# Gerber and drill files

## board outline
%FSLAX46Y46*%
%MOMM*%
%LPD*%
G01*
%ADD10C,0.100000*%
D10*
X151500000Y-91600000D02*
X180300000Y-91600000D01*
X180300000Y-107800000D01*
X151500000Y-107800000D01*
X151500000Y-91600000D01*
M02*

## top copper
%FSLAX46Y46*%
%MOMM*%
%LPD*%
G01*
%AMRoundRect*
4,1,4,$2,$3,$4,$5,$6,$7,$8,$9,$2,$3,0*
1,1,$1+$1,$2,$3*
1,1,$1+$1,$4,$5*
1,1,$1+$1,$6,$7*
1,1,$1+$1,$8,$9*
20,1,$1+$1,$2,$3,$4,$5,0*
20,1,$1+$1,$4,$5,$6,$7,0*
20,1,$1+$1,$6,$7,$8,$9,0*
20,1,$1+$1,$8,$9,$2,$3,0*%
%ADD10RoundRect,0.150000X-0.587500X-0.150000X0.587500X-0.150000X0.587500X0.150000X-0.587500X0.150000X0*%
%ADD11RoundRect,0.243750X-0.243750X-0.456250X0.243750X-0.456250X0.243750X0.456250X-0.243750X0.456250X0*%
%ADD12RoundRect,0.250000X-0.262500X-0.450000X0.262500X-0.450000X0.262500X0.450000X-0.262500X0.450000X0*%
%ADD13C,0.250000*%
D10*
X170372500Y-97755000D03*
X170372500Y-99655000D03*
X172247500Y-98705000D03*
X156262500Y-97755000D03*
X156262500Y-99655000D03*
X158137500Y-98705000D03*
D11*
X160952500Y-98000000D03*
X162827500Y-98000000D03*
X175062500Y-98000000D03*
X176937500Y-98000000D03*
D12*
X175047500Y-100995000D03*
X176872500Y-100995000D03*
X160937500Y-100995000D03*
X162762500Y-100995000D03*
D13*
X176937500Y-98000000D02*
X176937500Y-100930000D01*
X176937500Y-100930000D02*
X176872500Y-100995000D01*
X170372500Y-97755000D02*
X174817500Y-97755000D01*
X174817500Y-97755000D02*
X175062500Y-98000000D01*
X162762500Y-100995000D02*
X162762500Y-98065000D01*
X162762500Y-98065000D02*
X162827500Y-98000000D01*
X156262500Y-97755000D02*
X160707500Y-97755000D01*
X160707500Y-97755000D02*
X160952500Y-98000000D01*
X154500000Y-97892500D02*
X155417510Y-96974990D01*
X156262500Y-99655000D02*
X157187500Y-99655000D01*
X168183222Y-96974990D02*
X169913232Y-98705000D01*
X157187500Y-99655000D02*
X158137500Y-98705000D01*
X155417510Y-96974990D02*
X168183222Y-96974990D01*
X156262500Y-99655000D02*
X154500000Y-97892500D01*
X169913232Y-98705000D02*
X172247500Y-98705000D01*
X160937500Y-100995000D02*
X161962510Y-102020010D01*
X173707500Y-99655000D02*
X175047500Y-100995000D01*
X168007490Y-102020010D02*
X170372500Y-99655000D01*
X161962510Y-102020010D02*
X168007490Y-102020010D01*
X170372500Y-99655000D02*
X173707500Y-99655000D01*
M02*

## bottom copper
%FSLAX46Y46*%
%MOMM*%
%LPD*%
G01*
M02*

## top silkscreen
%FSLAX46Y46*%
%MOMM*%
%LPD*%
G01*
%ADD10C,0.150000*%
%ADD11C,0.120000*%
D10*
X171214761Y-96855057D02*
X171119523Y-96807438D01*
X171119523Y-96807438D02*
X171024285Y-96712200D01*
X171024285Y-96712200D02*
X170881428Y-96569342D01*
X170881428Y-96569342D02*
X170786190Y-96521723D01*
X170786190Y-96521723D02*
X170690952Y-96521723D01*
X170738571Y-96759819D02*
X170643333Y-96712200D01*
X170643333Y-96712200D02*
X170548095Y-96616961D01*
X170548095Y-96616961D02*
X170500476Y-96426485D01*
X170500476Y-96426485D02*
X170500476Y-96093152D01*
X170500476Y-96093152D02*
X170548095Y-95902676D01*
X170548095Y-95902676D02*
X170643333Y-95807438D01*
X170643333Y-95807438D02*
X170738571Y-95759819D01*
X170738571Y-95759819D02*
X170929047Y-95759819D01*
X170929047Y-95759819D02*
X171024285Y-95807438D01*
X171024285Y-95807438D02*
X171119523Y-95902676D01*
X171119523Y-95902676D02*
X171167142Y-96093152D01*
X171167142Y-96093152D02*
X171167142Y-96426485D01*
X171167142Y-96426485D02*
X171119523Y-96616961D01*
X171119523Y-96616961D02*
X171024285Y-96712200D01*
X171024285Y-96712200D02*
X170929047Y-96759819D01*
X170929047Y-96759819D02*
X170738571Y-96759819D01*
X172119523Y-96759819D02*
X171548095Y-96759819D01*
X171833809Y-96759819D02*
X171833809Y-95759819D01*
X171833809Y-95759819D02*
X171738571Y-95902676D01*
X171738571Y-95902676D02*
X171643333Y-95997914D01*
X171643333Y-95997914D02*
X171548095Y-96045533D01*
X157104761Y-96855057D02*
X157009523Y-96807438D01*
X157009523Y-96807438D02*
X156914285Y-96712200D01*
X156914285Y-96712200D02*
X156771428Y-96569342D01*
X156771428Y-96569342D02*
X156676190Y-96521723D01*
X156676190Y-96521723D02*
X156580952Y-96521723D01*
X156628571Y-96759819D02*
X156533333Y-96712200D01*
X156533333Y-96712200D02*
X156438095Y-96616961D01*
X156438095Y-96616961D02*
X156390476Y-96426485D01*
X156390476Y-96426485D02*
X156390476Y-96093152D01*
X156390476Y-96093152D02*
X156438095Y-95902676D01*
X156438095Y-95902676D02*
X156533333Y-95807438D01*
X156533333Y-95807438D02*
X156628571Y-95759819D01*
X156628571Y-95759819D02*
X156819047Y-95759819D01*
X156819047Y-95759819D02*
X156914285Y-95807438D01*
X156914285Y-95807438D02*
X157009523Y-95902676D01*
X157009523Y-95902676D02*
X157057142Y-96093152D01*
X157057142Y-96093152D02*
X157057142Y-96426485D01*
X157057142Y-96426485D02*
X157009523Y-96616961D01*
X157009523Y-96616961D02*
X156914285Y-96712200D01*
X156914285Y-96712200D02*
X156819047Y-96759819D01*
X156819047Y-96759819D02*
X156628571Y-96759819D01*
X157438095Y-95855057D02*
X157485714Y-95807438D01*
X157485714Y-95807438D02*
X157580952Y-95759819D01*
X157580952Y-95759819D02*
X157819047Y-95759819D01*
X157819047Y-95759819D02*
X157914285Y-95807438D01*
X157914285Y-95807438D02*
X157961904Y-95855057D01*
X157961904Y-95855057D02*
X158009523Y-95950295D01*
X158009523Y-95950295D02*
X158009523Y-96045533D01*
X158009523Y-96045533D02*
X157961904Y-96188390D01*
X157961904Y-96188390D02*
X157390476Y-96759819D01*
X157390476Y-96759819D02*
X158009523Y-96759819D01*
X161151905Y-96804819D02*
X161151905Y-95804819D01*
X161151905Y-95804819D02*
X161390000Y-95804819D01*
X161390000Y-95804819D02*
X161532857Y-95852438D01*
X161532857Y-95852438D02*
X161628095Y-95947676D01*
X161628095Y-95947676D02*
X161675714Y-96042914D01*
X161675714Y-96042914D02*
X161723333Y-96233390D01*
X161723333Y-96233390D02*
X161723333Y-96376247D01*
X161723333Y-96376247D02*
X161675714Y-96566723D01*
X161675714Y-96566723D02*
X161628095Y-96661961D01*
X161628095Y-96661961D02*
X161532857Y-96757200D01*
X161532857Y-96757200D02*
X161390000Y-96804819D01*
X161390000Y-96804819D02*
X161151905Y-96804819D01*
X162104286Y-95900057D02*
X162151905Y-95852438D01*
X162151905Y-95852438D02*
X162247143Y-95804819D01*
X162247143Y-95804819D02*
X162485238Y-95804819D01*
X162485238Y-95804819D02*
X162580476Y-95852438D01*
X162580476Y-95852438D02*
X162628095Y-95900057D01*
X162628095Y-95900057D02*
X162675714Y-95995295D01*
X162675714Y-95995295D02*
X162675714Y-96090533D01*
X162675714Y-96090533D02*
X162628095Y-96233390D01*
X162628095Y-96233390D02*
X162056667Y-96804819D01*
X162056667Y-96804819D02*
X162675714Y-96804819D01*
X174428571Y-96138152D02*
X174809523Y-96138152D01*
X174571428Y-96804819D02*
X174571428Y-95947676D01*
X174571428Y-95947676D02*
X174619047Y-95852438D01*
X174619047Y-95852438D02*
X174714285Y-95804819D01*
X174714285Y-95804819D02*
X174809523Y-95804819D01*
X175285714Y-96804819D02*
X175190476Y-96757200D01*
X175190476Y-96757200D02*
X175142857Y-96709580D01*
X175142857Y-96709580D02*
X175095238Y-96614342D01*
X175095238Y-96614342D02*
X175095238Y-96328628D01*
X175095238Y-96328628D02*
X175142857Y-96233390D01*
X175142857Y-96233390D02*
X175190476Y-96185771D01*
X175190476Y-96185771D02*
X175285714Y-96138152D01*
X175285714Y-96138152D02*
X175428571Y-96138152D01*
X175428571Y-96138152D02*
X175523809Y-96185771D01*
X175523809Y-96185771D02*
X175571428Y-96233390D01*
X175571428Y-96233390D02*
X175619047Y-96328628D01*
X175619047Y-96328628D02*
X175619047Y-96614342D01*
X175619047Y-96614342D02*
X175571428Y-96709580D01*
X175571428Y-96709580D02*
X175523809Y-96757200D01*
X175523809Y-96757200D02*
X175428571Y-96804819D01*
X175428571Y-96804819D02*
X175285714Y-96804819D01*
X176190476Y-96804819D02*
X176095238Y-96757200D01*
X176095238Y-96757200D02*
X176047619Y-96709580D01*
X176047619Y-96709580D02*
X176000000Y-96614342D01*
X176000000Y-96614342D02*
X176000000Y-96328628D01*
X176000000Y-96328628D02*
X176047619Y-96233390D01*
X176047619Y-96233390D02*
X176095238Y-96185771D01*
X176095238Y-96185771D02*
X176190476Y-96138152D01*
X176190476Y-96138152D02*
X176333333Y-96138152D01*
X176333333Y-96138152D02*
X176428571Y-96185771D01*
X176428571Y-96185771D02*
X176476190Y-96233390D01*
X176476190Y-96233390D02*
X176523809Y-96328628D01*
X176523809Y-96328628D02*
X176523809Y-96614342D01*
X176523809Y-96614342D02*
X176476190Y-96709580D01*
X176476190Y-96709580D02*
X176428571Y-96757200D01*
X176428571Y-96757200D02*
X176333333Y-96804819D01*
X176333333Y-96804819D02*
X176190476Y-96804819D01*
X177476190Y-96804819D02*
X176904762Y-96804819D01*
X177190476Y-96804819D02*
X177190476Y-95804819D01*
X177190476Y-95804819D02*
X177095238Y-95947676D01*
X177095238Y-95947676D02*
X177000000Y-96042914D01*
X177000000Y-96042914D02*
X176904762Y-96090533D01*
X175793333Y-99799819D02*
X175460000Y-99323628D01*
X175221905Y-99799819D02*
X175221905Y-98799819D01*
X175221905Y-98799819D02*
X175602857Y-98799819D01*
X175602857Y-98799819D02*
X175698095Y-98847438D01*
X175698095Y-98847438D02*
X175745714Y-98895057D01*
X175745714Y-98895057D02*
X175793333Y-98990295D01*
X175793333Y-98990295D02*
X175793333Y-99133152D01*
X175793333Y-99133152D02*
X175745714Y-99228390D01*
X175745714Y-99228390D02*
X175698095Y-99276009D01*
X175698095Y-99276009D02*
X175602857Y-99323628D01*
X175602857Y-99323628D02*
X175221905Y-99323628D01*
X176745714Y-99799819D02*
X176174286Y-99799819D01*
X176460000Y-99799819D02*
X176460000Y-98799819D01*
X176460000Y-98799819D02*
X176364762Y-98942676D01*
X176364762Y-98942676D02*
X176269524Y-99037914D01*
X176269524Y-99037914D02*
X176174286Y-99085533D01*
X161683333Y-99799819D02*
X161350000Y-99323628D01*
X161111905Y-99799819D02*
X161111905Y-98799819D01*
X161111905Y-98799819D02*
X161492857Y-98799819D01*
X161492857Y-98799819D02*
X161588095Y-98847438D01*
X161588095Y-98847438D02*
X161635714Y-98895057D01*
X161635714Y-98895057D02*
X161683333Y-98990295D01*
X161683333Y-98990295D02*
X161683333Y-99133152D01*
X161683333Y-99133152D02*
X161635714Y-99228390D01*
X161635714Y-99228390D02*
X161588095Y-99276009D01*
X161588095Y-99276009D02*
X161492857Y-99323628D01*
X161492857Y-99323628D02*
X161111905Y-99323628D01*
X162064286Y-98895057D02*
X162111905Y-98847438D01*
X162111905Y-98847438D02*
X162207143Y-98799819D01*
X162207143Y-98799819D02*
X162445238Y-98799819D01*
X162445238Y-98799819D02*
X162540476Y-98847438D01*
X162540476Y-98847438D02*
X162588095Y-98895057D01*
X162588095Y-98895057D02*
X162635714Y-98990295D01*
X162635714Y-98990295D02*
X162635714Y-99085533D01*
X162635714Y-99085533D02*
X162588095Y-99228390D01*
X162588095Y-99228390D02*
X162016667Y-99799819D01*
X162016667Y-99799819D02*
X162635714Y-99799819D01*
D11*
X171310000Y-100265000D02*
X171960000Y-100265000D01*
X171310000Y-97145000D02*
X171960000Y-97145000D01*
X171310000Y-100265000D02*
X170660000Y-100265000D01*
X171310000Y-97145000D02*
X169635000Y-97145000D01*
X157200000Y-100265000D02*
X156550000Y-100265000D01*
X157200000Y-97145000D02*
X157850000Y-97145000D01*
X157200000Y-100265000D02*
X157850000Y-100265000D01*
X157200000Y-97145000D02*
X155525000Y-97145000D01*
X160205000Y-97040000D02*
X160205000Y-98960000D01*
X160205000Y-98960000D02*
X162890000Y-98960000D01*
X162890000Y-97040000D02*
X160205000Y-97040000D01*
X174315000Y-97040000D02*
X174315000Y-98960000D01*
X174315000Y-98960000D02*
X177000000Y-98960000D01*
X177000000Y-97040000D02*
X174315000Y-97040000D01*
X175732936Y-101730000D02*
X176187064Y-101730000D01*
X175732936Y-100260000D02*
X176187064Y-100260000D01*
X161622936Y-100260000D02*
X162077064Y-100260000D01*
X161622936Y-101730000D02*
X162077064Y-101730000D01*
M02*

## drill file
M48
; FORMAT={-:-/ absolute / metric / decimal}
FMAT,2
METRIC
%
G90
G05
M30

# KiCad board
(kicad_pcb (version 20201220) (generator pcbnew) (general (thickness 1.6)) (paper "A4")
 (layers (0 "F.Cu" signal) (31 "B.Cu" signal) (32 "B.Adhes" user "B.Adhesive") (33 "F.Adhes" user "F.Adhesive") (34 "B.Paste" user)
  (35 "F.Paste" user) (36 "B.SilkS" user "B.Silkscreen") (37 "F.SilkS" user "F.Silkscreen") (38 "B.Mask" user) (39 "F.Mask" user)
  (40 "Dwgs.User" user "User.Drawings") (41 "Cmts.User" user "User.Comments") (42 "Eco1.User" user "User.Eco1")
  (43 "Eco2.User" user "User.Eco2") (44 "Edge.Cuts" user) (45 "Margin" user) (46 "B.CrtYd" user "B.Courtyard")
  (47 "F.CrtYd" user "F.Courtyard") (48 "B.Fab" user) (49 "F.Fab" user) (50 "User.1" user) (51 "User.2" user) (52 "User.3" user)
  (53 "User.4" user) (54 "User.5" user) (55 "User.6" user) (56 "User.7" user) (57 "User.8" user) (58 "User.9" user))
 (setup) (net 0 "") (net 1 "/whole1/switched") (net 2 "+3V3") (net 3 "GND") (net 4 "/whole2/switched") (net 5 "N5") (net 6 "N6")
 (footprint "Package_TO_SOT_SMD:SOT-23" (layer "F.Cu") (at 171.31 98.705)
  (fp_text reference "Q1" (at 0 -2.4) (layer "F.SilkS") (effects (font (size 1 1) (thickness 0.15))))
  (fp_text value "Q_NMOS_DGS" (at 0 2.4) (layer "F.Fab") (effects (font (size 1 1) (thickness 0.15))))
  (fp_line (start 0 1.56) (end 0.65 1.56) (layer "F.SilkS") (width 0.12))
  (fp_line (start 0 -1.56) (end 0.65 -1.56) (layer "F.SilkS") (width 0.12))
  (fp_line (start 0 1.56) (end -0.65 1.56) (layer "F.SilkS") (width 0.12))
  (fp_line (start 0 -1.56) (end -1.675 -1.56) (layer "F.SilkS") (width 0.12))
  (pad "1" smd roundrect (at -0.9375 -0.95) (size 1.475 0.6) (layers "F.Cu" "F.Paste" "F.Mask") (roundrect_rratio 0.25)
   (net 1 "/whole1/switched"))
  (pad "2" smd roundrect (at -0.9375 0.95) (size 1.475 0.6) (layers "F.Cu" "F.Paste" "F.Mask") (roundrect_rratio 0.25) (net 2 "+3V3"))
  (pad "3" smd roundrect (at 0.9375 0) (size 1.475 0.6) (layers "F.Cu" "F.Paste" "F.Mask") (roundrect_rratio 0.25) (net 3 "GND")))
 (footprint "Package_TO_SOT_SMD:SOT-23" (layer "F.Cu") (at 157.2 98.705)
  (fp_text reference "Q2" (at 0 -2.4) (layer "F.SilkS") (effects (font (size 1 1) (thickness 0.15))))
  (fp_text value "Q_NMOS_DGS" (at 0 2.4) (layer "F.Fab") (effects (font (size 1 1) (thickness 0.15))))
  (fp_line (start 0 1.56) (end -0.65 1.56) (layer "F.SilkS") (width 0.12))
  (fp_line (start 0 -1.56) (end 0.65 -1.56) (layer "F.SilkS") (width 0.12))
  (fp_line (start 0 1.56) (end 0.65 1.56) (layer "F.SilkS") (width 0.12))
  (fp_line (start 0 -1.56) (end -1.675 -1.56) (layer "F.SilkS") (width 0.12))
  (pad "1" smd roundrect (at -0.9375 -0.95) (size 1.475 0.6) (layers "F.Cu" "F.Paste" "F.Mask") (roundrect_rratio 0.25)
   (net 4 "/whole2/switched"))
  (pad "2" smd roundrect (at -0.9375 0.95) (size 1.475 0.6) (layers "F.Cu" "F.Paste" "F.Mask") (roundrect_rratio 0.25) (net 3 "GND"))
  (pad "3" smd roundrect (at 0.9375 0) (size 1.475 0.6) (layers "F.Cu" "F.Paste" "F.Mask") (roundrect_rratio 0.25) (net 3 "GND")))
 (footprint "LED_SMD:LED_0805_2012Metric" (layer "F.Cu") (at 161.89 98)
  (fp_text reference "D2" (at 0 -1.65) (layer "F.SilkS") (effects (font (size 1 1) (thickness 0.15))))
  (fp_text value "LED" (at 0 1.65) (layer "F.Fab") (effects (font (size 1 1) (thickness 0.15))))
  (fp_line (start -1.685 -0.96) (end -1.685 0.96) (layer "F.SilkS") (width 0.12))
  (fp_line (start -1.685 0.96) (end 1 0.96) (layer "F.SilkS") (width 0.12))
  (fp_line (start 1 -0.96) (end -1.685 -0.96) (layer "F.SilkS") (width 0.12))
  (pad "1" smd roundrect (at -0.9375 0) (size 0.975 1.4) (layers "F.Cu" "F.Paste" "F.Mask") (roundrect_rratio 0.25)
   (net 4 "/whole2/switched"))
  (pad "2" smd roundrect (at 0.9375 0) (size 0.975 1.4) (layers "F.Cu" "F.Paste" "F.Mask") (roundrect_rratio 0.25) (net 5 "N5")))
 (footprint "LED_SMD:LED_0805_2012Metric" (layer "F.Cu") (at 176 98)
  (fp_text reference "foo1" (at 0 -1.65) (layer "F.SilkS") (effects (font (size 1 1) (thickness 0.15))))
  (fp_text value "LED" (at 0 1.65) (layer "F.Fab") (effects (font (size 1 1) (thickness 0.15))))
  (fp_line (start -1.685 -0.96) (end -1.685 0.96) (layer "F.SilkS") (width 0.12))
  (fp_line (start -1.685 0.96) (end 1 0.96) (layer "F.SilkS") (width 0.12))
  (fp_line (start 1 -0.96) (end -1.685 -0.96) (layer "F.SilkS") (width 0.12))
  (pad "1" smd roundrect (at -0.9375 0) (size 0.975 1.4) (layers "F.Cu" "F.Paste" "F.Mask") (roundrect_rratio 0.25)
   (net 1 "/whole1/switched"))
  (pad "2" smd roundrect (at 0.9375 0) (size 0.975 1.4) (layers "F.Cu" "F.Paste" "F.Mask") (roundrect_rratio 0.25) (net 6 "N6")))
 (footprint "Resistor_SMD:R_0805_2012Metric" (layer "F.Cu") (at 175.96 100.995)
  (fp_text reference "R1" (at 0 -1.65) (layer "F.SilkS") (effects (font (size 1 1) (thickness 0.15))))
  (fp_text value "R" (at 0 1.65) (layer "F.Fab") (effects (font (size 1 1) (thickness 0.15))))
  (fp_line (start -0.227064 0.735) (end 0.227064 0.735) (layer "F.SilkS") (width 0.12))
  (fp_line (start -0.227064 -0.735) (end 0.227064 -0.735) (layer "F.SilkS") (width 0.12))
  (pad "1" smd roundrect (at -0.9125 0) (size 1.025 1.4) (layers "F.Cu" "F.Paste" "F.Mask") (roundrect_rratio 0.243902) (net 2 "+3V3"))
  (pad "2" smd roundrect (at 0.9125 0) (size 1.025 1.4) (layers "F.Cu" "F.Paste" "F.Mask") (roundrect_rratio 0.243902) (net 6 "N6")))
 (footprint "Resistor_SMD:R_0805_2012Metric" (layer "F.Cu") (at 161.85 100.995)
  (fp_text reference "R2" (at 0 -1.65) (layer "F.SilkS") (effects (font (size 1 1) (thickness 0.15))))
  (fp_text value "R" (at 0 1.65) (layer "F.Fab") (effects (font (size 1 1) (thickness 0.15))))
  (fp_line (start -0.227064 -0.735) (end 0.227064 -0.735) (layer "F.SilkS") (width 0.12))
  (fp_line (start -0.227064 0.735) (end 0.227064 0.735) (layer "F.SilkS") (width 0.12))
  (pad "1" smd roundrect (at -0.9125 0) (size 1.025 1.4) (layers "F.Cu" "F.Paste" "F.Mask") (roundrect_rratio 0.243902) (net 2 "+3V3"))
  (pad "2" smd roundrect (at 0.9125 0) (size 1.025 1.4) (layers "F.Cu" "F.Paste" "F.Mask") (roundrect_rratio 0.243902) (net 5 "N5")))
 (gr_rect (start 151.5 91.6) (end 180.3 107.8) (layer "Edge.Cuts") (width 0.1) (fill none))
 (segment (start 176.9375 98) (end 176.9375 100.93) (width 0.25) (layer "F.Cu") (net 6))
 (segment (start 176.9375 100.93) (end 176.8725 100.995) (width 0.25) (layer "F.Cu") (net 6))
 (segment (start 170.3725 97.755) (end 174.8175 97.755) (width 0.25) (layer "F.Cu") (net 1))
 (segment (start 174.8175 97.755) (end 175.0625 98) (width 0.25) (layer "F.Cu") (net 1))
 (segment (start 162.7625 100.995) (end 162.7625 98.065) (width 0.25) (layer "F.Cu") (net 5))
 (segment (start 162.7625 98.065) (end 162.8275 98) (width 0.25) (layer "F.Cu") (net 5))
 (segment (start 156.2625 97.755) (end 160.7075 97.755) (width 0.25) (layer "F.Cu") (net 4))
 (segment (start 160.7075 97.755) (end 160.9525 98) (width 0.25) (layer "F.Cu") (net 4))
 (segment (start 154.5 97.8925) (end 155.41751 96.97499) (width 0.25) (layer "F.Cu") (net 3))
 (segment (start 156.2625 99.655) (end 157.1875 99.655) (width 0.25) (layer "F.Cu") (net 3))
 (segment (start 168.183222 96.97499) (end 169.913232 98.705) (width 0.25) (layer "F.Cu") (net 3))
 (segment (start 157.1875 99.655) (end 158.1375 98.705) (width 0.25) (layer "F.Cu") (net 3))
 (segment (start 155.41751 96.97499) (end 168.183222 96.97499) (width 0.25) (layer "F.Cu") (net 3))
 (segment (start 156.2625 99.655) (end 154.5 97.8925) (width 0.25) (layer "F.Cu") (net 3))
 (segment (start 169.913232 98.705) (end 172.2475 98.705) (width 0.25) (layer "F.Cu") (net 3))
 (segment (start 160.9375 100.995) (end 161.96251 102.02001) (width 0.25) (layer "F.Cu") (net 2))
 (segment (start 173.7075 99.655) (end 175.0475 100.995) (width 0.25) (layer "F.Cu") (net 2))
 (segment (start 168.00749 102.02001) (end 170.3725 99.655) (width 0.25) (layer "F.Cu") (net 2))
 (segment (start 161.96251 102.02001) (end 168.00749 102.02001) (width 0.25) (layer "F.Cu") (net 2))
 (segment (start 170.3725 99.655) (end 173.7075 99.655) (width 0.25) (layer "F.Cu") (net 2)))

